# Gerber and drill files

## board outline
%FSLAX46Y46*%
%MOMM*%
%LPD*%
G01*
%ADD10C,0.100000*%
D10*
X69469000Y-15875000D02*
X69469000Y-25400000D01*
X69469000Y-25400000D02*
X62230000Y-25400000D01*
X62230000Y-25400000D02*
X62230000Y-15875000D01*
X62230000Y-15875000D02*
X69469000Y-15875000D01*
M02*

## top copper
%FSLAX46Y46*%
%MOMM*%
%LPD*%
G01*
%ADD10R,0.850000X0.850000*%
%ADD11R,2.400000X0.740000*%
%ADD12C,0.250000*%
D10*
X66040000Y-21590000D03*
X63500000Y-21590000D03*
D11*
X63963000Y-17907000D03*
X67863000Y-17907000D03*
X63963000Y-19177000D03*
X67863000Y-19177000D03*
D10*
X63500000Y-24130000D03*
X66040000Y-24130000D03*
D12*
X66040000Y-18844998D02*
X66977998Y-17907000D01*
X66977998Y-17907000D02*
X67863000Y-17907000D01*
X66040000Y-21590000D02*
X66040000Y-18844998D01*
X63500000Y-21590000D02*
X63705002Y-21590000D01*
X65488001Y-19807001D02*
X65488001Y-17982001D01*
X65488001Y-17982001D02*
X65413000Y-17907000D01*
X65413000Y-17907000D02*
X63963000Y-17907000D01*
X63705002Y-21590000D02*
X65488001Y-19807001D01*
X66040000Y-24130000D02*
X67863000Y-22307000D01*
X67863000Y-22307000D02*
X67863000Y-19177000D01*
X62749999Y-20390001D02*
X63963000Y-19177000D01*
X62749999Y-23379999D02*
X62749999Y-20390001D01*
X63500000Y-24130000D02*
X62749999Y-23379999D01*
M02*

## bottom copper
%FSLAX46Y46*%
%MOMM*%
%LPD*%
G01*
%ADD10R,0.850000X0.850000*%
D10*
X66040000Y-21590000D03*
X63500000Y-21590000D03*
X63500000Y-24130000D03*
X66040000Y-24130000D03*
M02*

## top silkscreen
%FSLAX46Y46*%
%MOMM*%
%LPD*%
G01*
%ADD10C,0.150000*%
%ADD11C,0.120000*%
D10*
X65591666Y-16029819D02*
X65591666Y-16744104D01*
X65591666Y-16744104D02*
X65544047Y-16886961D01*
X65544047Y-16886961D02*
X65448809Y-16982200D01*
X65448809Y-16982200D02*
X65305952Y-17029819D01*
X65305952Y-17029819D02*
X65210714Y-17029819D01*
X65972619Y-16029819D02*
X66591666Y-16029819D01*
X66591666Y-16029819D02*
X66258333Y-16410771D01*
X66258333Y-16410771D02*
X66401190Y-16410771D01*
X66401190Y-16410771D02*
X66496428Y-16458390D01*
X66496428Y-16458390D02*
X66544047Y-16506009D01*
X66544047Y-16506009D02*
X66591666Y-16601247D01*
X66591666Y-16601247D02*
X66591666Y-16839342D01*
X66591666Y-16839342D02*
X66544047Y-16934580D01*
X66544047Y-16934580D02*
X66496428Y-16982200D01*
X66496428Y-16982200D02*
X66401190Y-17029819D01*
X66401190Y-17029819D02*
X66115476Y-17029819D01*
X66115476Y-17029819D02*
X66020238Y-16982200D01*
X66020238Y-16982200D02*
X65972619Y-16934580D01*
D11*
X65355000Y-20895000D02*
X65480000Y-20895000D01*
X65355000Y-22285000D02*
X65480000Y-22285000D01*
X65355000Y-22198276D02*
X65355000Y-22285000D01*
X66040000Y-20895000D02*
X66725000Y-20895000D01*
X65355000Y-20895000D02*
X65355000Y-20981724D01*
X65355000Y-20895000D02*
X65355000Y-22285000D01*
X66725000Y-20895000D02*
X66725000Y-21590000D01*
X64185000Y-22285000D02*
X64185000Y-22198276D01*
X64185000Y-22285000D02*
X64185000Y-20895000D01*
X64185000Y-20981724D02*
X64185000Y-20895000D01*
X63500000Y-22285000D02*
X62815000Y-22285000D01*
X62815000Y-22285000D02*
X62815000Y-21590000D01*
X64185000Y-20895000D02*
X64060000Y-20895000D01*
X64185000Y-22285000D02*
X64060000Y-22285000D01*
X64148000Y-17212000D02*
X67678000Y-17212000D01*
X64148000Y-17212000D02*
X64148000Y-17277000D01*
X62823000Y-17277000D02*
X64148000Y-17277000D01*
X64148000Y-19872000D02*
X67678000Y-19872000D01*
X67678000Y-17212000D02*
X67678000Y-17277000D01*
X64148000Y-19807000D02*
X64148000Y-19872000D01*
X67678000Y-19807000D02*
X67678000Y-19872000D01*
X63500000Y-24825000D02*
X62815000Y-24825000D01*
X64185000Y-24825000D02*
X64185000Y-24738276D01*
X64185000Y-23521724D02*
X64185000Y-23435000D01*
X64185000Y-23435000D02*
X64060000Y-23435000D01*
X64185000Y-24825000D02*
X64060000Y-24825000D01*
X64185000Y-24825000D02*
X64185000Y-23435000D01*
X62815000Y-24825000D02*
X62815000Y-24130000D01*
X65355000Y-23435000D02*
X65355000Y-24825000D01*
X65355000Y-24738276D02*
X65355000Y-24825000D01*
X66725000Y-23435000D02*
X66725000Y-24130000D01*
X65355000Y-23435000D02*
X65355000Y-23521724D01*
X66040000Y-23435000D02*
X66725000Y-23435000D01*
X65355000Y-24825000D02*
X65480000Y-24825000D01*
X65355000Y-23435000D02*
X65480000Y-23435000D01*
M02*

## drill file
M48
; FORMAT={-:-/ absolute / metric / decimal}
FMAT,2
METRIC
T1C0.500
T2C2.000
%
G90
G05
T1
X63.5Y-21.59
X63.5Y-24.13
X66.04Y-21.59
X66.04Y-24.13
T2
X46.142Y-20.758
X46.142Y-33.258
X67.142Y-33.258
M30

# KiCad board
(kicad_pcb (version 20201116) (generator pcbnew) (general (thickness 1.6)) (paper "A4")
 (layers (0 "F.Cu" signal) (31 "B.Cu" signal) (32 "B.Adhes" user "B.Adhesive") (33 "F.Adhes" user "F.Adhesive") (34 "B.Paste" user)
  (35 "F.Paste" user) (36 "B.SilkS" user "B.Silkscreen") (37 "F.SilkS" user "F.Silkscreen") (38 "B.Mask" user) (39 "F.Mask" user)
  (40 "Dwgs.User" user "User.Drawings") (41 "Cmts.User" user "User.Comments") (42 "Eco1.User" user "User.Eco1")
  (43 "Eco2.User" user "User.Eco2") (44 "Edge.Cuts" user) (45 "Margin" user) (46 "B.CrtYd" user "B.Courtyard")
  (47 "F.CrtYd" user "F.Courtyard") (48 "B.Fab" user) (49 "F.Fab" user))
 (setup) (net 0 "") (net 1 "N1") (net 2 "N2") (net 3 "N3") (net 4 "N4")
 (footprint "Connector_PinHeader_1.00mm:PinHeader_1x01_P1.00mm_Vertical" (layer "F.Cu") (at 66.04 21.59 -90)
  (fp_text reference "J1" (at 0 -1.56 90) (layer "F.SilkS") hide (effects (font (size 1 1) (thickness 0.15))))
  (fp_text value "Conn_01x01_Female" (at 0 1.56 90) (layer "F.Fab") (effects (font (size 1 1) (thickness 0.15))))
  (fp_line (start -0.695 0.685) (end -0.695 0.56) (layer "F.SilkS") (width 0.12))
  (fp_line (start 0.695 0.685) (end 0.695 0.56) (layer "F.SilkS") (width 0.12))
  (fp_line (start 0.608276 0.685) (end 0.695 0.685) (layer "F.SilkS") (width 0.12))
  (fp_line (start -0.695 0) (end -0.695 -0.685) (layer "F.SilkS") (width 0.12))
  (fp_line (start -0.695 0.685) (end -0.608276 0.685) (layer "F.SilkS") (width 0.12))
  (fp_line (start -0.695 0.685) (end 0.695 0.685) (layer "F.SilkS") (width 0.12))
  (fp_line (start -0.695 -0.685) (end 0 -0.685) (layer "F.SilkS") (width 0.12))
  (pad "1" thru_hole rect (at 0 0 270) (size 0.85 0.85) (drill 0.5) (layers *.Cu *.Mask) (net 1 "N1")))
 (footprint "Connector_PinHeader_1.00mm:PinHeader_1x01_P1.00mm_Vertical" (layer "F.Cu") (at 63.5 21.59 90)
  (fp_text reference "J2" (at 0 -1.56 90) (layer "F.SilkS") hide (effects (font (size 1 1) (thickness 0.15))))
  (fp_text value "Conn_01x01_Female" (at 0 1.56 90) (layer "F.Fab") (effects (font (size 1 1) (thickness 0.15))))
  (fp_line (start -0.695 0.685) (end -0.608276 0.685) (layer "F.SilkS") (width 0.12))
  (fp_line (start -0.695 0.685) (end 0.695 0.685) (layer "F.SilkS") (width 0.12))
  (fp_line (start 0.608276 0.685) (end 0.695 0.685) (layer "F.SilkS") (width 0.12))
  (fp_line (start -0.695 0) (end -0.695 -0.685) (layer "F.SilkS") (width 0.12))
  (fp_line (start -0.695 -0.685) (end 0 -0.685) (layer "F.SilkS") (width 0.12))
  (fp_line (start 0.695 0.685) (end 0.695 0.56) (layer "F.SilkS") (width 0.12))
  (fp_line (start -0.695 0.685) (end -0.695 0.56) (layer "F.SilkS") (width 0.12))
  (pad "1" thru_hole rect (at 0 0 90) (size 0.85 0.85) (drill 0.5) (layers *.Cu *.Mask) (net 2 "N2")))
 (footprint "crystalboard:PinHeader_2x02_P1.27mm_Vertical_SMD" (layer "F.Cu") (at 65.913 18.542)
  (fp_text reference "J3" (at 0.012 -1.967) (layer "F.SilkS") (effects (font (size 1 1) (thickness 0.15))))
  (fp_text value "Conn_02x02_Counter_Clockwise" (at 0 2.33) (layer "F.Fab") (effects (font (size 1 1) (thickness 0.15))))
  (fp_line (start -1.765 -1.33) (end 1.765 -1.33) (layer "F.SilkS") (width 0.12))
  (fp_line (start -1.765 -1.33) (end -1.765 -1.265) (layer "F.SilkS") (width 0.12))
  (fp_line (start -3.09 -1.265) (end -1.765 -1.265) (layer "F.SilkS") (width 0.12))
  (fp_line (start -1.765 1.33) (end 1.765 1.33) (layer "F.SilkS") (width 0.12))
  (fp_line (start 1.765 -1.33) (end 1.765 -1.265) (layer "F.SilkS") (width 0.12))
  (fp_line (start -1.765 1.265) (end -1.765 1.33) (layer "F.SilkS") (width 0.12))
  (fp_line (start 1.765 1.265) (end 1.765 1.33) (layer "F.SilkS") (width 0.12))
  (pad "1" smd rect (at -1.95 -0.635) (size 2.4 0.74) (layers "F.Cu" "F.Paste" "F.Mask") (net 2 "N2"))
  (pad "2" smd rect (at 1.95 -0.635) (size 2.4 0.74) (layers "F.Cu" "F.Paste" "F.Mask") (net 1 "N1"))
  (pad "3" smd rect (at -1.95 0.635) (size 2.4 0.74) (layers "F.Cu" "F.Paste" "F.Mask") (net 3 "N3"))
  (pad "4" smd rect (at 1.95 0.635) (size 2.4 0.74) (layers "F.Cu" "F.Paste" "F.Mask") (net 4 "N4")))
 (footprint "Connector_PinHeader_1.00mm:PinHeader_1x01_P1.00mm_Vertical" (layer "F.Cu") (at 63.5 24.13 90)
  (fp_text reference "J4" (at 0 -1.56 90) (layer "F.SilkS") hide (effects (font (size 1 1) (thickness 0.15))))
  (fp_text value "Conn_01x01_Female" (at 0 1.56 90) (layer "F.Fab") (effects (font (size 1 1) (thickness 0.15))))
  (fp_line (start -0.695 0) (end -0.695 -0.685) (layer "F.SilkS") (width 0.12))
  (fp_line (start -0.695 0.685) (end -0.608276 0.685) (layer "F.SilkS") (width 0.12))
  (fp_line (start 0.608276 0.685) (end 0.695 0.685) (layer "F.SilkS") (width 0.12))
  (fp_line (start 0.695 0.685) (end 0.695 0.56) (layer "F.SilkS") (width 0.12))
  (fp_line (start -0.695 0.685) (end -0.695 0.56) (layer "F.SilkS") (width 0.12))
  (fp_line (start -0.695 0.685) (end 0.695 0.685) (layer "F.SilkS") (width 0.12))
  (fp_line (start -0.695 -0.685) (end 0 -0.685) (layer "F.SilkS") (width 0.12))
  (pad "1" thru_hole rect (at 0 0 90) (size 0.85 0.85) (drill 0.5) (layers *.Cu *.Mask) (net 3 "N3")))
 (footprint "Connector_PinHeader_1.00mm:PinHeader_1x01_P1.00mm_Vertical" (layer "F.Cu") (at 66.04 24.13 -90)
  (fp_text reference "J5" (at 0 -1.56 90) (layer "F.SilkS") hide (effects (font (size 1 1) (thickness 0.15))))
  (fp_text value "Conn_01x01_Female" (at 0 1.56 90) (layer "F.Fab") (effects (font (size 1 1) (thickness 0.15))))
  (fp_line (start -0.695 0.685) (end 0.695 0.685) (layer "F.SilkS") (width 0.12))
  (fp_line (start 0.608276 0.685) (end 0.695 0.685) (layer "F.SilkS") (width 0.12))
  (fp_line (start -0.695 -0.685) (end 0 -0.685) (layer "F.SilkS") (width 0.12))
  (fp_line (start -0.695 0.685) (end -0.608276 0.685) (layer "F.SilkS") (width 0.12))
  (fp_line (start -0.695 0) (end -0.695 -0.685) (layer "F.SilkS") (width 0.12))
  (fp_line (start 0.695 0.685) (end 0.695 0.56) (layer "F.SilkS") (width 0.12))
  (fp_line (start -0.695 0.685) (end -0.695 0.56) (layer "F.SilkS") (width 0.12))
  (pad "1" thru_hole rect (at 0 0 270) (size 0.85 0.85) (drill 0.5) (layers *.Cu *.Mask) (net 4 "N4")))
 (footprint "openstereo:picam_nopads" (layer "B.Cu") (at 56.642 32.258 180)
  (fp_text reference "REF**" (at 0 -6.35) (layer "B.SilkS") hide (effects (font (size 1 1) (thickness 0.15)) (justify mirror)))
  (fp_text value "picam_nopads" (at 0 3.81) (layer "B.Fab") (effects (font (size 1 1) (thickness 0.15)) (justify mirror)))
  (pad "" np_thru_hole circle (at 10.5 11.5 180) (size 2 2) (drill 2) (layers *.Cu *.Mask))
  (pad "" np_thru_hole circle (at -10.5 -1 180) (size 2 2) (drill 2) (layers *.Cu *.Mask))
  (pad "" np_thru_hole circle (at 10.5 -1 180) (size 2 2) (drill 2) (layers *.Cu *.Mask)))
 (gr_line (start 69.469 15.875) (end 69.469 25.4) (layer "Edge.Cuts") (width 0.1))
 (gr_line (start 69.469 25.4) (end 62.23 25.4) (layer "Edge.Cuts") (width 0.1))
 (gr_line (start 62.23 25.4) (end 62.23 15.875) (layer "Edge.Cuts") (width 0.1))
 (gr_line (start 62.23 15.875) (end 69.469 15.875) (layer "Edge.Cuts") (width 0.1))
 (segment (start 66.04 18.844998) (end 66.977998 17.907) (width 0.25) (layer "F.Cu") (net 1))
 (segment (start 66.977998 17.907) (end 67.863 17.907) (width 0.25) (layer "F.Cu") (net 1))
 (segment (start 66.04 21.59) (end 66.04 18.844998) (width 0.25) (layer "F.Cu") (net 1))
 (segment (start 63.5 21.59) (end 63.705002 21.59) (width 0.25) (layer "F.Cu") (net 2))
 (segment (start 65.488001 19.807001) (end 65.488001 17.982001) (width 0.25) (layer "F.Cu") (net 2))
 (segment (start 65.488001 17.982001) (end 65.413 17.907) (width 0.25) (layer "F.Cu") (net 2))
 (segment (start 65.413 17.907) (end 63.963 17.907) (width 0.25) (layer "F.Cu") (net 2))
 (segment (start 63.705002 21.59) (end 65.488001 19.807001) (width 0.25) (layer "F.Cu") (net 2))
 (segment (start 66.04 24.13) (end 67.863 22.307) (width 0.25) (layer "F.Cu") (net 4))
 (segment (start 67.863 22.307) (end 67.863 19.177) (width 0.25) (layer "F.Cu") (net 4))
 (segment (start 62.749999 20.390001) (end 63.963 19.177) (width 0.25) (layer "F.Cu") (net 3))
 (segment (start 62.749999 23.379999) (end 62.749999 20.390001) (width 0.25) (layer "F.Cu") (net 3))
 (segment (start 63.5 24.13) (end 62.749999 23.379999) (width 0.25) (layer "F.Cu") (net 3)))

